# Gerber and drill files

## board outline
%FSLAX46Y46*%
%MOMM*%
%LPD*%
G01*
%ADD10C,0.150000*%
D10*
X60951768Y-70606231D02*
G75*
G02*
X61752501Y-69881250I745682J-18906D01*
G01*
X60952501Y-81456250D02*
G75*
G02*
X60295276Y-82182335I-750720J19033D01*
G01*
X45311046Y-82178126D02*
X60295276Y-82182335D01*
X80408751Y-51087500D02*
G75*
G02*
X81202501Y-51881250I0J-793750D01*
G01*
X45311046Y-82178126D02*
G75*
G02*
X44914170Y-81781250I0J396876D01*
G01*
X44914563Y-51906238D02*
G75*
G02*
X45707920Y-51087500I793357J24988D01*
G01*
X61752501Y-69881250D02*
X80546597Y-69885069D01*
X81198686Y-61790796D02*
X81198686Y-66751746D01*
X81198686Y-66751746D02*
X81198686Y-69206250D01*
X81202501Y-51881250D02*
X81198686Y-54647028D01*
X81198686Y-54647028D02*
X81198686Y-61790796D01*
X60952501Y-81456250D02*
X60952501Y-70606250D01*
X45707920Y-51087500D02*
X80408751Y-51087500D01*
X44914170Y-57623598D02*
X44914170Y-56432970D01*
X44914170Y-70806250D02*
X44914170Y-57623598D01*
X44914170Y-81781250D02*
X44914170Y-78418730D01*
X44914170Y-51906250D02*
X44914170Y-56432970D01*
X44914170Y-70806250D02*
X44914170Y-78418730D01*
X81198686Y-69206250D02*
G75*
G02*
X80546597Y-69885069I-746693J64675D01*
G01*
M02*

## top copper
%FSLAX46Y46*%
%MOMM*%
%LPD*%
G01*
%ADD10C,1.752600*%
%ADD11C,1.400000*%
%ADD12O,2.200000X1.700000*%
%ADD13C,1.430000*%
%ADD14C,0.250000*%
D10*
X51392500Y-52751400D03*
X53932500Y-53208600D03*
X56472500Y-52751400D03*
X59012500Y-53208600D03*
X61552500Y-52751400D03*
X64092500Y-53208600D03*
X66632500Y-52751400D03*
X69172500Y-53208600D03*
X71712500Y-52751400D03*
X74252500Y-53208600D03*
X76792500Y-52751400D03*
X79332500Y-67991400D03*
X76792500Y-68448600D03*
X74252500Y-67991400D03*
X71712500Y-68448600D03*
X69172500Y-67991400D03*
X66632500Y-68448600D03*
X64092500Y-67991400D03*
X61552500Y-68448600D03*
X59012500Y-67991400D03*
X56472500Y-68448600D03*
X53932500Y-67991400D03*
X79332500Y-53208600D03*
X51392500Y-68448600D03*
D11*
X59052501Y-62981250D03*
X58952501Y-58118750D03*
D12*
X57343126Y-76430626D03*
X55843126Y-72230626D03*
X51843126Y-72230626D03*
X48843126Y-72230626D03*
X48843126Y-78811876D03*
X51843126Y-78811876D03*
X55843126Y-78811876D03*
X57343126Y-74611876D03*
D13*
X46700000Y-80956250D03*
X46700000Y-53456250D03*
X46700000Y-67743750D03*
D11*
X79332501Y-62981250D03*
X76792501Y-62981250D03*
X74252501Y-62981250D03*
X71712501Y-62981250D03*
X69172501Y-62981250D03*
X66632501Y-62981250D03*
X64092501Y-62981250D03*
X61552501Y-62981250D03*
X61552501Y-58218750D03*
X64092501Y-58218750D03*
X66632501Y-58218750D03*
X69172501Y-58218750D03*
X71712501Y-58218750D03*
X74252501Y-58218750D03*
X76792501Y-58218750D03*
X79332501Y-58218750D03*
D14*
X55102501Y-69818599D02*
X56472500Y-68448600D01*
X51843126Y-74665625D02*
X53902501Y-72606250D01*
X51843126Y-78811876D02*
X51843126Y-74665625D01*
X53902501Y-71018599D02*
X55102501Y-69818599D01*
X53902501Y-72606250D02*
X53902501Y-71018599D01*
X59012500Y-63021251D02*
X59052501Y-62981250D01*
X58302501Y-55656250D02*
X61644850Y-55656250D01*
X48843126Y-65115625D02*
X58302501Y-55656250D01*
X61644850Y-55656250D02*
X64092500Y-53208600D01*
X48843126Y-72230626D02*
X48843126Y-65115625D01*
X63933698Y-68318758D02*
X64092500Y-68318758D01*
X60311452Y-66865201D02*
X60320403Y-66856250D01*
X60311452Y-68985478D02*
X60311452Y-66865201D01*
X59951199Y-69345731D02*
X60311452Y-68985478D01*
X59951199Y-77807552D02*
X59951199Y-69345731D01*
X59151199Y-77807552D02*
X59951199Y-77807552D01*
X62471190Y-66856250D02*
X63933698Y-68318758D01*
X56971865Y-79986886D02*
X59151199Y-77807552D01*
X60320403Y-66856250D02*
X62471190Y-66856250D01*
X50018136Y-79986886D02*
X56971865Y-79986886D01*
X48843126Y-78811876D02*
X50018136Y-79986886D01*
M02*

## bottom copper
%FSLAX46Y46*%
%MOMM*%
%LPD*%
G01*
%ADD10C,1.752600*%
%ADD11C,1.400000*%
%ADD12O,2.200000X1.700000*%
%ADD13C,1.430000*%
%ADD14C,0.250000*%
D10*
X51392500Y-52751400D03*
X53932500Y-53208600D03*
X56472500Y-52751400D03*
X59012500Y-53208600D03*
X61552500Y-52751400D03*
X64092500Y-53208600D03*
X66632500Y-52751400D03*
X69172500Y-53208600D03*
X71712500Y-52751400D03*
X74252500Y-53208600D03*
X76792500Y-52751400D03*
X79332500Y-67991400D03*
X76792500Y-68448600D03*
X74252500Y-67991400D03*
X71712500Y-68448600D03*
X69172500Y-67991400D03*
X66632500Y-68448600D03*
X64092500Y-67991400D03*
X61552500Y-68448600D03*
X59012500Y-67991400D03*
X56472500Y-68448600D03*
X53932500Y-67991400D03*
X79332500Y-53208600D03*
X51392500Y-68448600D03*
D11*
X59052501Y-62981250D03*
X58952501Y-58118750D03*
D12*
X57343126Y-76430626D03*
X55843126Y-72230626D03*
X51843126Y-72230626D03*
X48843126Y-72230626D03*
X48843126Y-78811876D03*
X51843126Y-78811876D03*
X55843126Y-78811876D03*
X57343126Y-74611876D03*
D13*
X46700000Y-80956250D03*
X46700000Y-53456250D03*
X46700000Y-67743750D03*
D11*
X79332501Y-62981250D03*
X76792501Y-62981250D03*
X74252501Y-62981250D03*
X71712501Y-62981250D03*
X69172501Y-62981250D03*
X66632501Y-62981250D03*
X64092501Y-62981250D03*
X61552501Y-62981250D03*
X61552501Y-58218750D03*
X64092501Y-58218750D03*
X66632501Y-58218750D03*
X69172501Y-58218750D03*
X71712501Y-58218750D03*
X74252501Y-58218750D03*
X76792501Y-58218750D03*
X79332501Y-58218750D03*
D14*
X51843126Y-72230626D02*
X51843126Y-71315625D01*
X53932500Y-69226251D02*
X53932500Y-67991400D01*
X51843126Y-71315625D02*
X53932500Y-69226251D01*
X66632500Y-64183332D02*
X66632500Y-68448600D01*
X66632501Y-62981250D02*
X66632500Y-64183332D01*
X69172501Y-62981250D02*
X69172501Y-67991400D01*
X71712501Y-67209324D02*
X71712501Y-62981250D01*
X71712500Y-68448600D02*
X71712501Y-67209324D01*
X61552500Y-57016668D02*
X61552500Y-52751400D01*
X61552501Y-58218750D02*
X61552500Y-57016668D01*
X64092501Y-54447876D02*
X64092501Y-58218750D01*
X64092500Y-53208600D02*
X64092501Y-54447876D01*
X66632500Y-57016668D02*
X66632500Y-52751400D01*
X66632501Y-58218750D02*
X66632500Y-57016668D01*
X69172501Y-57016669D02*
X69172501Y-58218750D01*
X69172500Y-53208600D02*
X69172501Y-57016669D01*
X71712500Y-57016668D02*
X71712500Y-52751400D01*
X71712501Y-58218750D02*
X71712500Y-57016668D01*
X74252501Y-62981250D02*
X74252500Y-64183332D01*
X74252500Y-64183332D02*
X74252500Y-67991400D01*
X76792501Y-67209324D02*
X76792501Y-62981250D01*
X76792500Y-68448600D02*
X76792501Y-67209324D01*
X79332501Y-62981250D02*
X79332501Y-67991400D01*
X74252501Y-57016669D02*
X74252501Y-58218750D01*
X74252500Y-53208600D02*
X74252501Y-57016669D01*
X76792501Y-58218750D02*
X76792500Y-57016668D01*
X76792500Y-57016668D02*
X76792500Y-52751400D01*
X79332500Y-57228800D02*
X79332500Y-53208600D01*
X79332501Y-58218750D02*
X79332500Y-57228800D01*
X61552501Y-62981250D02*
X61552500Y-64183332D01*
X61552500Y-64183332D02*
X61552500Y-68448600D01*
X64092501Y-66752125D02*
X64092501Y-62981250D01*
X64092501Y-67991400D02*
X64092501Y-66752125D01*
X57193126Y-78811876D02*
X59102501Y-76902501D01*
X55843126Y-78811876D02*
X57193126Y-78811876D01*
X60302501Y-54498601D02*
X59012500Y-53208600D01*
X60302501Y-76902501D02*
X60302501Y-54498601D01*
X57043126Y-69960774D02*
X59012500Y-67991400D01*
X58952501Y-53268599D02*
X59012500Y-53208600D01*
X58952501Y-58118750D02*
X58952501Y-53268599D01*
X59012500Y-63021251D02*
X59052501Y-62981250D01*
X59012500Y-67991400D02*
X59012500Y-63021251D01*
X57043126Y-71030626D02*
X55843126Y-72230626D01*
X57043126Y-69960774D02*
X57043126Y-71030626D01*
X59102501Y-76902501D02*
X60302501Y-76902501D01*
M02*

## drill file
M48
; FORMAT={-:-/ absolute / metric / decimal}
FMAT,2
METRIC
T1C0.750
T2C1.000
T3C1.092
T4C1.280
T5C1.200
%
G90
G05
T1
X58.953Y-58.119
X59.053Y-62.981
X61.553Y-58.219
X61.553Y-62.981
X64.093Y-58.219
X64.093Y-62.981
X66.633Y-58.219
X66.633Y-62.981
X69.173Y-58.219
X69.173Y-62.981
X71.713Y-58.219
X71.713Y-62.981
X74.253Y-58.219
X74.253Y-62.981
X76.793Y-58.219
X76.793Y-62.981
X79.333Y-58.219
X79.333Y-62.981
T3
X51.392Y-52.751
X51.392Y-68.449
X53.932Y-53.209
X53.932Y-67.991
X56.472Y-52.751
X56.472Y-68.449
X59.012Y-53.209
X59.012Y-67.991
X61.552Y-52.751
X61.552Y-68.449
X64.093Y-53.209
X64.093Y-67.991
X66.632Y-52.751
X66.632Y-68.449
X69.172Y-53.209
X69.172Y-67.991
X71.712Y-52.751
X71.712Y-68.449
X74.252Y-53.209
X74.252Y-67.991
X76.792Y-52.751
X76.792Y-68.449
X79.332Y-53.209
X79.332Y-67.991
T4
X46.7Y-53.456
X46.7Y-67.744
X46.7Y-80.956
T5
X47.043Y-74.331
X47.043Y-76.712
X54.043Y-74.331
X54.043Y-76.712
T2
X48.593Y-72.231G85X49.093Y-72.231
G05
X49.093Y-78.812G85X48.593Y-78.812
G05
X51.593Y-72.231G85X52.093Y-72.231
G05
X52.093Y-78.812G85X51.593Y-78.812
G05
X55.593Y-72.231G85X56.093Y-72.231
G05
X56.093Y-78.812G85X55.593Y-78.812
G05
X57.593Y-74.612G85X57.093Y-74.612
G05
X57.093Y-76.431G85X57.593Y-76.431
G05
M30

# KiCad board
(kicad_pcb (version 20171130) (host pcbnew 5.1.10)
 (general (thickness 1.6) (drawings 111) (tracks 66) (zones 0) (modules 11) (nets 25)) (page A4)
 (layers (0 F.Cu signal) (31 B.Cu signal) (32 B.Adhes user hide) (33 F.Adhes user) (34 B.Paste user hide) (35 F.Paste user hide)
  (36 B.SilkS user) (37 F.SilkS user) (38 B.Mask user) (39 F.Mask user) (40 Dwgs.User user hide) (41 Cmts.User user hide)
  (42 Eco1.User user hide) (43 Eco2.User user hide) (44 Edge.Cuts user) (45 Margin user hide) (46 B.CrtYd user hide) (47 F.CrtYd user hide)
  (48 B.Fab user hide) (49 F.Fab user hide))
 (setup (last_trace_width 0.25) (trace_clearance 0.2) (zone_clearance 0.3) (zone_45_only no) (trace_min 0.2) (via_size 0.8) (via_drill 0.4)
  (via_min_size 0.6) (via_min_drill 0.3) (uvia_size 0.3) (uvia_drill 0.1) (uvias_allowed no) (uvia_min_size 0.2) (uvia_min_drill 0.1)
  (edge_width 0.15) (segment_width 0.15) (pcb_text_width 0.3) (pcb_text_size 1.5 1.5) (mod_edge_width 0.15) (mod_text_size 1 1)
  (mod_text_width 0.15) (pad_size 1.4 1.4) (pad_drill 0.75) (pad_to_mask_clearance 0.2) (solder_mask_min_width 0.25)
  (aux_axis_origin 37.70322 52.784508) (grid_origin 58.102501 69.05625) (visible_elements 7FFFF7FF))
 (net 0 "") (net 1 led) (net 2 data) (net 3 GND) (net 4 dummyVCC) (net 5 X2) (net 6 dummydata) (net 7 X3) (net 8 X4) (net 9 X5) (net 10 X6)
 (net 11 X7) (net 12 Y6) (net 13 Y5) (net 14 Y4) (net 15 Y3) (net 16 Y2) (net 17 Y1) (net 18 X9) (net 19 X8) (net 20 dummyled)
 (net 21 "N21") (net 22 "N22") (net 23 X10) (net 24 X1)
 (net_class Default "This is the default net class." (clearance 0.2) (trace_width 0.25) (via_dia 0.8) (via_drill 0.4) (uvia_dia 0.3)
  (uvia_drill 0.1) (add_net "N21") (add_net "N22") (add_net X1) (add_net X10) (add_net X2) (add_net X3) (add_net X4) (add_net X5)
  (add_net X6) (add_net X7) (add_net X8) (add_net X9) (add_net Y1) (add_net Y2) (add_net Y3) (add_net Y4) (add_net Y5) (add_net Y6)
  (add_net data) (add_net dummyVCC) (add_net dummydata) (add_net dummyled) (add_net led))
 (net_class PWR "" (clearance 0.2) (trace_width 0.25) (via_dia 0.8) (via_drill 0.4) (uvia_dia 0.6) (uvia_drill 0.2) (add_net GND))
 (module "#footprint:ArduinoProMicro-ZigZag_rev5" (layer B.Cu) (at 65.3625 60.6)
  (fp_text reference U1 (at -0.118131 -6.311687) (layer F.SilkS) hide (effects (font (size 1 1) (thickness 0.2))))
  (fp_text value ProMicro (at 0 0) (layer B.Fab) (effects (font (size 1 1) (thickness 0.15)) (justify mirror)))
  (pad 1 thru_hole circle (at -13.97 -7.8486) (size 1.7526 1.7526) (drill 1.0922) (layers *.Cu *.SilkS *.Mask) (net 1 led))
  (pad 2 thru_hole circle (at -11.43 -7.3914) (size 1.7526 1.7526) (drill 1.0922) (layers *.Cu *.SilkS *.Mask) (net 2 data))
  (pad 3 thru_hole circle (at -8.89 -7.8486) (size 1.7526 1.7526) (drill 1.0922) (layers *.Cu *.SilkS *.Mask) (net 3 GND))
  (pad 4 thru_hole circle (at -6.35 -7.3914) (size 1.7526 1.7526) (drill 1.0922) (layers *.Cu *.SilkS *.Mask) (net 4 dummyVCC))
  (pad 5 thru_hole circle (at -3.81 -7.8486) (size 1.7526 1.7526) (drill 1.0922) (layers *.Cu *.SilkS *.Mask) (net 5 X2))
  (pad 6 thru_hole circle (at -1.27 -7.3914) (size 1.7526 1.7526) (drill 1.0922) (layers *.Cu *.SilkS *.Mask) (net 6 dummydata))
  (pad 7 thru_hole circle (at 1.27 -7.8486) (size 1.7526 1.7526) (drill 1.0922) (layers *.Cu *.SilkS *.Mask) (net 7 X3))
  (pad 8 thru_hole circle (at 3.81 -7.3914) (size 1.7526 1.7526) (drill 1.0922) (layers *.Cu *.SilkS *.Mask) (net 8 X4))
  (pad 9 thru_hole circle (at 6.35 -7.8486) (size 1.7526 1.7526) (drill 1.0922) (layers *.Cu *.SilkS *.Mask) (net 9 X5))
  (pad 10 thru_hole circle (at 8.89 -7.3914) (size 1.7526 1.7526) (drill 1.0922) (layers *.Cu *.SilkS *.Mask) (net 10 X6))
  (pad 11 thru_hole circle (at 11.43 -7.8486) (size 1.7526 1.7526) (drill 1.0922) (layers *.Cu *.SilkS *.Mask) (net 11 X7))
  (pad 13 thru_hole circle (at 13.97 7.3914) (size 1.7526 1.7526) (drill 1.0922) (layers *.Cu *.SilkS *.Mask) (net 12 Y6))
  (pad 14 thru_hole circle (at 11.43 7.8486) (size 1.7526 1.7526) (drill 1.0922) (layers *.Cu *.SilkS *.Mask) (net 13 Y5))
  (pad 15 thru_hole circle (at 8.89 7.3914) (size 1.7526 1.7526) (drill 1.0922) (layers *.Cu *.SilkS *.Mask) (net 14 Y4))
  (pad 16 thru_hole circle (at 6.35 7.8486) (size 1.7526 1.7526) (drill 1.0922) (layers *.Cu *.SilkS *.Mask) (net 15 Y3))
  (pad 17 thru_hole circle (at 3.81 7.3914) (size 1.7526 1.7526) (drill 1.0922) (layers *.Cu *.SilkS *.Mask) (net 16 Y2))
  (pad 18 thru_hole circle (at 1.27 7.8486) (size 1.7526 1.7526) (drill 1.0922) (layers *.Cu *.SilkS *.Mask) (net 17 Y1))
  (pad 19 thru_hole circle (at -1.27 7.3914) (size 1.7526 1.7526) (drill 1.0922) (layers *.Cu *.SilkS *.Mask) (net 6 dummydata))
  (pad 20 thru_hole circle (at -3.81 7.8486) (size 1.7526 1.7526) (drill 1.0922) (layers *.Cu *.SilkS *.Mask) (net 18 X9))
  (pad 21 thru_hole circle (at -6.35 7.3914) (size 1.7526 1.7526) (drill 1.0922) (layers *.Cu *.SilkS *.Mask) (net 4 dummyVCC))
  (pad 22 thru_hole circle (at -8.89 7.8486) (size 1.7526 1.7526) (drill 1.0922) (layers *.Cu *.SilkS *.Mask) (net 3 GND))
  (pad 23 thru_hole circle (at -11.43 7.3914) (size 1.7526 1.7526) (drill 1.0922) (layers *.Cu *.SilkS *.Mask) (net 3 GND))
  (pad 12 thru_hole circle (at 13.97 -7.3914) (size 1.7526 1.7526) (drill 1.0922) (layers *.Cu *.SilkS *.Mask) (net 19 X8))
  (pad 24 thru_hole circle (at -13.97 7.8486) (size 1.7526 1.7526) (drill 1.0922) (layers *.Cu *.SilkS *.Mask) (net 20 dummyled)))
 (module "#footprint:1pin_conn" (layer F.Cu) (at 59.052501 63.00625) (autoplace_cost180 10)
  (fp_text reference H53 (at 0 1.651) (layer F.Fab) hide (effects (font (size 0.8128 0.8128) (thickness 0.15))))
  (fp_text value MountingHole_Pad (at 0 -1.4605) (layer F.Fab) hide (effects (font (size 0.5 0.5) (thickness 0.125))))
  (pad 1 thru_hole circle (at 0 -0.025) (size 1.4 1.4) (drill 0.75) (layers *.Cu *.Mask) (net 4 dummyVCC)))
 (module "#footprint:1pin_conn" (layer F.Cu) (at 58.952501 58.21875) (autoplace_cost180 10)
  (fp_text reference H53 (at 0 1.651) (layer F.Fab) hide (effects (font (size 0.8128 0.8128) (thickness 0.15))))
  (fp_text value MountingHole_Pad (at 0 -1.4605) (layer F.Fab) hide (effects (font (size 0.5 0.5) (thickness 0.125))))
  (pad 1 thru_hole circle (at 0 -0.1) (size 1.4 1.4) (drill 0.75) (layers *.Cu *.Mask) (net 4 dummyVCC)))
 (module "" (layer F.Cu) (at 8.552501 -16.34375)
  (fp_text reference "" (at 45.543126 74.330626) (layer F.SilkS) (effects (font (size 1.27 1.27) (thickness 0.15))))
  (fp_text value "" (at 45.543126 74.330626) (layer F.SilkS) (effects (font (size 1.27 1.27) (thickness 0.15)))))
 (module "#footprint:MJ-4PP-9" (layer F.Cu) (at 45.543126 74.330626 90)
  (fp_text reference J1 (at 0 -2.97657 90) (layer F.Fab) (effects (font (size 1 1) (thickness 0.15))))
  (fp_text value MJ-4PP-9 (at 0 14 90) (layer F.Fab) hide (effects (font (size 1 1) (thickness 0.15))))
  (pad A thru_hole oval (at -2.1 11.8 90) (size 1.7 2.2) (drill oval 1 1.5) (layers *.Cu *.Mask F.SilkS) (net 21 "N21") (clearance 0.15))
  (pad D thru_hole oval (at 2.1 10.3 90) (size 1.7 2.2) (drill oval 1 1.5) (layers *.Cu *.Mask F.SilkS) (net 4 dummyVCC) (clearance 0.15))
  (pad C thru_hole oval (at 2.1 6.3 90) (size 1.7 2.2) (drill oval 1 1.5) (layers *.Cu *.Mask F.SilkS) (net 3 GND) (clearance 0.15))
  (pad B thru_hole oval (at 2.1 3.3 90) (size 1.7 2.2) (drill oval 1 1.5) (layers *.Cu *.Mask F.SilkS) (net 6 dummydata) (clearance 0.15))
  (pad "" np_thru_hole circle (at 0 8.5 90) (size 1.2 1.2) (drill 1.2) (layers *.Cu *.Mask F.SilkS))
  (pad "" np_thru_hole circle (at 0 1.5 90) (size 1.2 1.2) (drill 1.2) (layers *.Cu *.Mask F.SilkS)))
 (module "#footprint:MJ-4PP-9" (layer B.Cu) (at 45.543126 76.711876 270)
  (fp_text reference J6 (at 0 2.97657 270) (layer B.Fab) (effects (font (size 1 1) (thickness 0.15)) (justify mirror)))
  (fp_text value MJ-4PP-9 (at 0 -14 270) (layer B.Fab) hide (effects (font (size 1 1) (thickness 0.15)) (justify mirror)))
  (pad "" np_thru_hole circle (at 0 -1.5 270) (size 1.2 1.2) (drill 1.2) (layers *.Cu *.Mask B.SilkS))
  (pad "" np_thru_hole circle (at 0 -8.5 270) (size 1.2 1.2) (drill 1.2) (layers *.Cu *.Mask B.SilkS))
  (pad B thru_hole oval (at 2.1 -3.3 270) (size 1.7 2.2) (drill oval 1 1.5) (layers *.Cu *.Mask B.SilkS) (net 6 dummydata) (clearance 0.15))
  (pad C thru_hole oval (at 2.1 -6.3 270) (size 1.7 2.2) (drill oval 1 1.5) (layers *.Cu *.Mask B.SilkS) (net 3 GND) (clearance 0.15))
  (pad D thru_hole oval (at 2.1 -10.3 270) (size 1.7 2.2) (drill oval 1 1.5) (layers *.Cu *.Mask B.SilkS) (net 4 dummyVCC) (clearance 0.15))
  (pad A thru_hole oval (at -2.1 -11.8 270) (size 1.7 2.2) (drill oval 1 1.5) (layers *.Cu *.Mask B.SilkS) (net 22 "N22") (clearance 0.15)))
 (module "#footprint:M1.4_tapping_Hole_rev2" (layer F.Cu) (at 46.102501 80.95625) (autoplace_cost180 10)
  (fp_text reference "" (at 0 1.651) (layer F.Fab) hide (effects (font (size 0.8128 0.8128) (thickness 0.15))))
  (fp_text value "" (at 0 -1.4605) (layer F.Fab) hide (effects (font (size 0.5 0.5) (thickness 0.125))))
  (pad "" thru_hole circle (at 0.597499 0) (size 1.43 1.43) (drill 1.28) (layers *.Cu *.Mask)))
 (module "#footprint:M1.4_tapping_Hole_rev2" (layer F.Cu) (at 46.7 53.45625) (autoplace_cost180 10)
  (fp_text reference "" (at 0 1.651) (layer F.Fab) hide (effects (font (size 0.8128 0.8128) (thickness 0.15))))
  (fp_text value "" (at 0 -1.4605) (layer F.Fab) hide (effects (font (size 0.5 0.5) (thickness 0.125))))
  (pad "" thru_hole circle (at 0 0) (size 1.43 1.43) (drill 1.28) (layers *.Cu *.Mask)))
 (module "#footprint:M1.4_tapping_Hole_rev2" (layer F.Cu) (at 46.7 67.74375) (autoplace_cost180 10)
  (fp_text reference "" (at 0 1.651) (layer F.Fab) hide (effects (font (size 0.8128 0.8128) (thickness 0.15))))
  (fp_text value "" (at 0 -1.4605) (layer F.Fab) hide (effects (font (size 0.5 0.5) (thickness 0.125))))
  (pad "" thru_hole circle (at 0 0) (size 1.43 1.43) (drill 1.28) (layers *.Cu *.Mask)))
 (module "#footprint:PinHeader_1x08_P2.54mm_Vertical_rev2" (layer F.Cu) (at 61.552501 62.98125 90)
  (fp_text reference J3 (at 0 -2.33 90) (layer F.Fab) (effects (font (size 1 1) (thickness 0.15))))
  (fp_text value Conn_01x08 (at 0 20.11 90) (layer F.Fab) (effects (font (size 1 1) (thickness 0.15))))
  (pad 8 thru_hole circle (at 0 17.78 90) (size 1.4 1.4) (drill 0.75) (layers *.Cu *.Mask) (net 12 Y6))
  (pad 7 thru_hole circle (at 0 15.24 90) (size 1.4 1.4) (drill 0.75) (layers *.Cu *.Mask) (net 13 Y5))
  (pad 6 thru_hole circle (at 0 12.7 90) (size 1.4 1.4) (drill 0.75) (layers *.Cu *.Mask) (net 14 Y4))
  (pad 5 thru_hole circle (at 0 10.16 90) (size 1.4 1.4) (drill 0.75) (layers *.Cu *.Mask) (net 15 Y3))
  (pad 4 thru_hole circle (at 0 7.62 90) (size 1.4 1.4) (drill 0.75) (layers *.Cu *.Mask) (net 16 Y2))
  (pad 3 thru_hole circle (at 0 5.08 90) (size 1.4 1.4) (drill 0.75) (layers *.Cu *.Mask) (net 17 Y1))
  (pad 2 thru_hole circle (at 0 2.54 90) (size 1.4 1.4) (drill 0.75) (layers *.Cu *.Mask) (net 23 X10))
  (pad 1 thru_hole circle (at 0 0 90) (size 1.4 1.4) (drill 0.75) (layers *.Cu *.Mask) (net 18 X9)))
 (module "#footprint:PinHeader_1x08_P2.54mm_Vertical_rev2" (layer F.Cu) (at 61.552501 58.21875 90)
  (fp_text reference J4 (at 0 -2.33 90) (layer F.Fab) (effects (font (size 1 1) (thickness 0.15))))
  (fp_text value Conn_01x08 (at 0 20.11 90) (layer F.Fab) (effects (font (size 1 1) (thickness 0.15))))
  (pad 1 thru_hole circle (at 0 0 90) (size 1.4 1.4) (drill 0.75) (layers *.Cu *.Mask) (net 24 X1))
  (pad 2 thru_hole circle (at 0 2.54 90) (size 1.4 1.4) (drill 0.75) (layers *.Cu *.Mask) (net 5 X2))
  (pad 3 thru_hole circle (at 0 5.08 90) (size 1.4 1.4) (drill 0.75) (layers *.Cu *.Mask) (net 7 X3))
  (pad 4 thru_hole circle (at 0 7.62 90) (size 1.4 1.4) (drill 0.75) (layers *.Cu *.Mask) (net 8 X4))
  (pad 5 thru_hole circle (at 0 10.16 90) (size 1.4 1.4) (drill 0.75) (layers *.Cu *.Mask) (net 9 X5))
  (pad 6 thru_hole circle (at 0 12.7 90) (size 1.4 1.4) (drill 0.75) (layers *.Cu *.Mask) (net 10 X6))
  (pad 7 thru_hole circle (at 0 15.24 90) (size 1.4 1.4) (drill 0.75) (layers *.Cu *.Mask) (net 11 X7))
  (pad 8 thru_hole circle (at 0 17.78 90) (size 1.4 1.4) (drill 0.75) (layers *.Cu *.Mask) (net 19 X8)))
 (gr_arc (start 61.69745 70.625137) (end 61.752501 69.88125) (angle -92.78006695) (layer Edge.Cuts) (width 0.15))
 (gr_arc (start 60.201781 81.437217) (end 60.295276 82.182335) (angle -81.39578011) (layer Edge.Cuts) (width 0.15))
 (gr_line (start 45.311046 82.178126) (end 60.295276 82.182335) (layer Edge.Cuts) (width 0.15))
 (gr_arc (start 80.408751 51.88125) (end 81.202501 51.88125) (angle -90) (layer Edge.Cuts) (width 0.15))
 (gr_arc (start 45.311046 81.78125) (end 44.91417 81.78125) (angle -90) (layer Edge.Cuts) (width 0.15))
 (gr_arc (start 45.70792 51.88125) (end 45.70792 51.0875) (angle -91.80399512) (layer Edge.Cuts) (width 0.15))
 (gr_line (start 61.752501 69.88125) (end 80.546597 69.885069) (layer Edge.Cuts) (width 0.15))
 (gr_line (start 81.198686 61.790796) (end 81.198686 66.751746) (layer Edge.Cuts) (width 0.15))
 (gr_line (start 81.198686 66.751746) (end 81.198686 69.20625) (layer Edge.Cuts) (width 0.15))
 (gr_line (start 81.202501 51.88125) (end 81.198686 54.647028) (layer Edge.Cuts) (width 0.15))
 (gr_line (start 81.198686 54.647028) (end 81.198686 61.790796) (layer Edge.Cuts) (width 0.15))
 (gr_line (start 60.952501 81.45625) (end 60.952501 70.60625) (layer Edge.Cuts) (width 0.15))
 (gr_line (start 45.70792 51.0875) (end 80.408751 51.0875) (layer Edge.Cuts) (width 0.15))
 (gr_line (start 44.91417 57.623598) (end 44.91417 56.43297) (layer Edge.Cuts) (width 0.15))
 (gr_line (start 44.91417 70.80625) (end 44.91417 57.623598) (layer Edge.Cuts) (width 0.15))
 (gr_line (start 44.91417 81.78125) (end 44.91417 78.41873) (layer Edge.Cuts) (width 0.15))
 (gr_line (start 44.91417 51.90625) (end 44.91417 56.43297) (layer Edge.Cuts) (width 0.15))
 (gr_line (start 44.91417 70.80625) (end 44.91417 78.41873) (layer Edge.Cuts) (width 0.15))
 (gr_arc (start 80.451993 69.141575) (end 80.546597 69.885069) (angle -77.79817896) (layer Edge.Cuts) (width 0.15))
 (segment (start 55.102501 69.818599) (end 56.4725 68.4486) (width 0.25) (layer F.Cu) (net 3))
 (segment (start 51.843126 74.665625) (end 53.902501 72.60625) (width 0.25) (layer F.Cu) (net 3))
 (segment (start 51.843126 78.811876) (end 51.843126 74.665625) (width 0.25) (layer F.Cu) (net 3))
 (segment (start 53.902501 71.018599) (end 55.102501 69.818599) (width 0.25) (layer F.Cu) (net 3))
 (segment (start 53.902501 72.60625) (end 53.902501 71.018599) (width 0.25) (layer F.Cu) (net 3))
 (segment (start 51.843126 72.230626) (end 51.843126 71.315625) (width 0.25) (layer B.Cu) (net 3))
 (segment (start 53.9325 69.226251) (end 53.9325 67.9914) (width 0.25) (layer B.Cu) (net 3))
 (segment (start 51.843126 71.315625) (end 53.9325 69.226251) (width 0.25) (layer B.Cu) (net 3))
 (segment (start 66.6325 64.183332) (end 66.6325 68.4486) (width 0.25) (layer B.Cu) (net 17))
 (segment (start 66.632501 62.98125) (end 66.6325 64.183332) (width 0.25) (layer B.Cu) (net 17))
 (segment (start 69.172501 62.98125) (end 69.172501 67.9914) (width 0.25) (layer B.Cu) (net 16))
 (segment (start 71.712501 67.209324) (end 71.712501 62.98125) (width 0.25) (layer B.Cu) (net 15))
 (segment (start 71.7125 68.4486) (end 71.712501 67.209324) (width 0.25) (layer B.Cu) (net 15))
 (segment (start 61.5525 57.016668) (end 61.5525 52.7514) (width 0.25) (layer B.Cu) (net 24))
 (segment (start 61.552501 58.21875) (end 61.5525 57.016668) (width 0.25) (layer B.Cu) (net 24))
 (segment (start 64.092501 54.447876) (end 64.092501 58.21875) (width 0.25) (layer B.Cu) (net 5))
 (segment (start 64.0925 53.2086) (end 64.092501 54.447876) (width 0.25) (layer B.Cu) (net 5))
 (segment (start 66.6325 57.016668) (end 66.6325 52.7514) (width 0.25) (layer B.Cu) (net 7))
 (segment (start 66.632501 58.21875) (end 66.6325 57.016668) (width 0.25) (layer B.Cu) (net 7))
 (segment (start 69.172501 57.016669) (end 69.172501 58.21875) (width 0.25) (layer B.Cu) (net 8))
 (segment (start 69.1725 53.2086) (end 69.172501 57.016669) (width 0.25) (layer B.Cu) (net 8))
 (segment (start 71.7125 57.016668) (end 71.7125 52.7514) (width 0.25) (layer B.Cu) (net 9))
 (segment (start 71.712501 58.21875) (end 71.7125 57.016668) (width 0.25) (layer B.Cu) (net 9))
 (segment (start 74.252501 62.98125) (end 74.2525 64.183332) (width 0.25) (layer B.Cu) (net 14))
 (segment (start 74.2525 64.183332) (end 74.2525 67.9914) (width 0.25) (layer B.Cu) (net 14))
 (segment (start 76.792501 67.209324) (end 76.792501 62.98125) (width 0.25) (layer B.Cu) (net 13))
 (segment (start 76.7925 68.4486) (end 76.792501 67.209324) (width 0.25) (layer B.Cu) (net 13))
 (segment (start 79.332501 62.98125) (end 79.332501 67.9914) (width 0.25) (layer B.Cu) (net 12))
 (segment (start 74.252501 57.016669) (end 74.252501 58.21875) (width 0.25) (layer B.Cu) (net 10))
 (segment (start 74.2525 53.2086) (end 74.252501 57.016669) (width 0.25) (layer B.Cu) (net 10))
 (segment (start 76.792501 58.21875) (end 76.7925 57.016668) (width 0.25) (layer B.Cu) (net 11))
 (segment (start 76.7925 57.016668) (end 76.7925 52.7514) (width 0.25) (layer B.Cu) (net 11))
 (segment (start 79.3325 57.2288) (end 79.3325 53.2086) (width 0.25) (layer B.Cu) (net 19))
 (segment (start 79.332501 58.21875) (end 79.3325 57.2288) (width 0.25) (layer B.Cu) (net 19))
 (segment (start 61.552501 62.98125) (end 61.5525 64.183332) (width 0.25) (layer B.Cu) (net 18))
 (segment (start 61.5525 64.183332) (end 61.5525 68.4486) (width 0.25) (layer B.Cu) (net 18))
 (segment (start 64.092501 66.752125) (end 64.092501 62.98125) (width 0.25) (layer B.Cu) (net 23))
 (segment (start 64.092501 67.9914) (end 64.092501 66.752125) (width 0.25) (layer B.Cu) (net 23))
 (segment (start 57.193126 78.811876) (end 59.102501 76.902501) (width 0.25) (layer B.Cu) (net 4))
 (segment (start 55.843126 78.811876) (end 57.193126 78.811876) (width 0.25) (layer B.Cu) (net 4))
 (segment (start 60.302501 54.498601) (end 59.0125 53.2086) (width 0.25) (layer B.Cu) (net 4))
 (segment (start 60.302501 76.902501) (end 60.302501 54.498601) (width 0.25) (layer B.Cu) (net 4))
 (segment (start 57.043126 69.960774) (end 59.0125 67.9914) (width 0.25) (layer B.Cu) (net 4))
 (segment (start 58.952501 53.268599) (end 59.0125 53.2086) (width 0.25) (layer B.Cu) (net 4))
 (segment (start 58.952501 58.11875) (end 58.952501 53.268599) (width 0.25) (layer B.Cu) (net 4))
 (segment (start 59.0125 63.021251) (end 59.052501 62.98125) (width 0.25) (layer F.Cu) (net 4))
 (segment (start 59.0125 63.021251) (end 59.052501 62.98125) (width 0.25) (layer B.Cu) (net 4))
 (segment (start 59.0125 67.9914) (end 59.0125 63.021251) (width 0.25) (layer B.Cu) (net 4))
 (segment (start 57.043126 71.030626) (end 55.843126 72.230626) (width 0.25) (layer B.Cu) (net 4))
 (segment (start 57.043126 69.960774) (end 57.043126 71.030626) (width 0.25) (layer B.Cu) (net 4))
 (segment (start 59.102501 76.902501) (end 60.302501 76.902501) (width 0.25) (layer B.Cu) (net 4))
 (segment (start 58.302501 55.65625) (end 61.64485 55.65625) (width 0.25) (layer F.Cu) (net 6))
 (segment (start 48.843126 65.115625) (end 58.302501 55.65625) (width 0.25) (layer F.Cu) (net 6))
 (segment (start 61.64485 55.65625) (end 64.0925 53.2086) (width 0.25) (layer F.Cu) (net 6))
 (segment (start 48.843126 72.230626) (end 48.843126 65.115625) (width 0.25) (layer F.Cu) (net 6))
 (segment (start 63.933698 68.318758) (end 64.0925 68.318758) (width 0.25) (layer F.Cu) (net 6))
 (segment (start 60.311452 66.865201) (end 60.320403 66.85625) (width 0.25) (layer F.Cu) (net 6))
 (segment (start 60.311452 68.985478) (end 60.311452 66.865201) (width 0.25) (layer F.Cu) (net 6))
 (segment (start 59.951199 69.345731) (end 60.311452 68.985478) (width 0.25) (layer F.Cu) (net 6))
 (segment (start 59.951199 77.807552) (end 59.951199 69.345731) (width 0.25) (layer F.Cu) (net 6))
 (segment (start 59.151199 77.807552) (end 59.951199 77.807552) (width 0.25) (layer F.Cu) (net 6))
 (segment (start 62.47119 66.85625) (end 63.933698 68.318758) (width 0.25) (layer F.Cu) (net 6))
 (segment (start 56.971865 79.986886) (end 59.151199 77.807552) (width 0.25) (layer F.Cu) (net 6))
 (segment (start 60.320403 66.85625) (end 62.47119 66.85625) (width 0.25) (layer F.Cu) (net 6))
 (segment (start 50.018136 79.986886) (end 56.971865 79.986886) (width 0.25) (layer F.Cu) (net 6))
 (segment (start 48.843126 78.811876) (end 50.018136 79.986886) (width 0.25) (layer F.Cu) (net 6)))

